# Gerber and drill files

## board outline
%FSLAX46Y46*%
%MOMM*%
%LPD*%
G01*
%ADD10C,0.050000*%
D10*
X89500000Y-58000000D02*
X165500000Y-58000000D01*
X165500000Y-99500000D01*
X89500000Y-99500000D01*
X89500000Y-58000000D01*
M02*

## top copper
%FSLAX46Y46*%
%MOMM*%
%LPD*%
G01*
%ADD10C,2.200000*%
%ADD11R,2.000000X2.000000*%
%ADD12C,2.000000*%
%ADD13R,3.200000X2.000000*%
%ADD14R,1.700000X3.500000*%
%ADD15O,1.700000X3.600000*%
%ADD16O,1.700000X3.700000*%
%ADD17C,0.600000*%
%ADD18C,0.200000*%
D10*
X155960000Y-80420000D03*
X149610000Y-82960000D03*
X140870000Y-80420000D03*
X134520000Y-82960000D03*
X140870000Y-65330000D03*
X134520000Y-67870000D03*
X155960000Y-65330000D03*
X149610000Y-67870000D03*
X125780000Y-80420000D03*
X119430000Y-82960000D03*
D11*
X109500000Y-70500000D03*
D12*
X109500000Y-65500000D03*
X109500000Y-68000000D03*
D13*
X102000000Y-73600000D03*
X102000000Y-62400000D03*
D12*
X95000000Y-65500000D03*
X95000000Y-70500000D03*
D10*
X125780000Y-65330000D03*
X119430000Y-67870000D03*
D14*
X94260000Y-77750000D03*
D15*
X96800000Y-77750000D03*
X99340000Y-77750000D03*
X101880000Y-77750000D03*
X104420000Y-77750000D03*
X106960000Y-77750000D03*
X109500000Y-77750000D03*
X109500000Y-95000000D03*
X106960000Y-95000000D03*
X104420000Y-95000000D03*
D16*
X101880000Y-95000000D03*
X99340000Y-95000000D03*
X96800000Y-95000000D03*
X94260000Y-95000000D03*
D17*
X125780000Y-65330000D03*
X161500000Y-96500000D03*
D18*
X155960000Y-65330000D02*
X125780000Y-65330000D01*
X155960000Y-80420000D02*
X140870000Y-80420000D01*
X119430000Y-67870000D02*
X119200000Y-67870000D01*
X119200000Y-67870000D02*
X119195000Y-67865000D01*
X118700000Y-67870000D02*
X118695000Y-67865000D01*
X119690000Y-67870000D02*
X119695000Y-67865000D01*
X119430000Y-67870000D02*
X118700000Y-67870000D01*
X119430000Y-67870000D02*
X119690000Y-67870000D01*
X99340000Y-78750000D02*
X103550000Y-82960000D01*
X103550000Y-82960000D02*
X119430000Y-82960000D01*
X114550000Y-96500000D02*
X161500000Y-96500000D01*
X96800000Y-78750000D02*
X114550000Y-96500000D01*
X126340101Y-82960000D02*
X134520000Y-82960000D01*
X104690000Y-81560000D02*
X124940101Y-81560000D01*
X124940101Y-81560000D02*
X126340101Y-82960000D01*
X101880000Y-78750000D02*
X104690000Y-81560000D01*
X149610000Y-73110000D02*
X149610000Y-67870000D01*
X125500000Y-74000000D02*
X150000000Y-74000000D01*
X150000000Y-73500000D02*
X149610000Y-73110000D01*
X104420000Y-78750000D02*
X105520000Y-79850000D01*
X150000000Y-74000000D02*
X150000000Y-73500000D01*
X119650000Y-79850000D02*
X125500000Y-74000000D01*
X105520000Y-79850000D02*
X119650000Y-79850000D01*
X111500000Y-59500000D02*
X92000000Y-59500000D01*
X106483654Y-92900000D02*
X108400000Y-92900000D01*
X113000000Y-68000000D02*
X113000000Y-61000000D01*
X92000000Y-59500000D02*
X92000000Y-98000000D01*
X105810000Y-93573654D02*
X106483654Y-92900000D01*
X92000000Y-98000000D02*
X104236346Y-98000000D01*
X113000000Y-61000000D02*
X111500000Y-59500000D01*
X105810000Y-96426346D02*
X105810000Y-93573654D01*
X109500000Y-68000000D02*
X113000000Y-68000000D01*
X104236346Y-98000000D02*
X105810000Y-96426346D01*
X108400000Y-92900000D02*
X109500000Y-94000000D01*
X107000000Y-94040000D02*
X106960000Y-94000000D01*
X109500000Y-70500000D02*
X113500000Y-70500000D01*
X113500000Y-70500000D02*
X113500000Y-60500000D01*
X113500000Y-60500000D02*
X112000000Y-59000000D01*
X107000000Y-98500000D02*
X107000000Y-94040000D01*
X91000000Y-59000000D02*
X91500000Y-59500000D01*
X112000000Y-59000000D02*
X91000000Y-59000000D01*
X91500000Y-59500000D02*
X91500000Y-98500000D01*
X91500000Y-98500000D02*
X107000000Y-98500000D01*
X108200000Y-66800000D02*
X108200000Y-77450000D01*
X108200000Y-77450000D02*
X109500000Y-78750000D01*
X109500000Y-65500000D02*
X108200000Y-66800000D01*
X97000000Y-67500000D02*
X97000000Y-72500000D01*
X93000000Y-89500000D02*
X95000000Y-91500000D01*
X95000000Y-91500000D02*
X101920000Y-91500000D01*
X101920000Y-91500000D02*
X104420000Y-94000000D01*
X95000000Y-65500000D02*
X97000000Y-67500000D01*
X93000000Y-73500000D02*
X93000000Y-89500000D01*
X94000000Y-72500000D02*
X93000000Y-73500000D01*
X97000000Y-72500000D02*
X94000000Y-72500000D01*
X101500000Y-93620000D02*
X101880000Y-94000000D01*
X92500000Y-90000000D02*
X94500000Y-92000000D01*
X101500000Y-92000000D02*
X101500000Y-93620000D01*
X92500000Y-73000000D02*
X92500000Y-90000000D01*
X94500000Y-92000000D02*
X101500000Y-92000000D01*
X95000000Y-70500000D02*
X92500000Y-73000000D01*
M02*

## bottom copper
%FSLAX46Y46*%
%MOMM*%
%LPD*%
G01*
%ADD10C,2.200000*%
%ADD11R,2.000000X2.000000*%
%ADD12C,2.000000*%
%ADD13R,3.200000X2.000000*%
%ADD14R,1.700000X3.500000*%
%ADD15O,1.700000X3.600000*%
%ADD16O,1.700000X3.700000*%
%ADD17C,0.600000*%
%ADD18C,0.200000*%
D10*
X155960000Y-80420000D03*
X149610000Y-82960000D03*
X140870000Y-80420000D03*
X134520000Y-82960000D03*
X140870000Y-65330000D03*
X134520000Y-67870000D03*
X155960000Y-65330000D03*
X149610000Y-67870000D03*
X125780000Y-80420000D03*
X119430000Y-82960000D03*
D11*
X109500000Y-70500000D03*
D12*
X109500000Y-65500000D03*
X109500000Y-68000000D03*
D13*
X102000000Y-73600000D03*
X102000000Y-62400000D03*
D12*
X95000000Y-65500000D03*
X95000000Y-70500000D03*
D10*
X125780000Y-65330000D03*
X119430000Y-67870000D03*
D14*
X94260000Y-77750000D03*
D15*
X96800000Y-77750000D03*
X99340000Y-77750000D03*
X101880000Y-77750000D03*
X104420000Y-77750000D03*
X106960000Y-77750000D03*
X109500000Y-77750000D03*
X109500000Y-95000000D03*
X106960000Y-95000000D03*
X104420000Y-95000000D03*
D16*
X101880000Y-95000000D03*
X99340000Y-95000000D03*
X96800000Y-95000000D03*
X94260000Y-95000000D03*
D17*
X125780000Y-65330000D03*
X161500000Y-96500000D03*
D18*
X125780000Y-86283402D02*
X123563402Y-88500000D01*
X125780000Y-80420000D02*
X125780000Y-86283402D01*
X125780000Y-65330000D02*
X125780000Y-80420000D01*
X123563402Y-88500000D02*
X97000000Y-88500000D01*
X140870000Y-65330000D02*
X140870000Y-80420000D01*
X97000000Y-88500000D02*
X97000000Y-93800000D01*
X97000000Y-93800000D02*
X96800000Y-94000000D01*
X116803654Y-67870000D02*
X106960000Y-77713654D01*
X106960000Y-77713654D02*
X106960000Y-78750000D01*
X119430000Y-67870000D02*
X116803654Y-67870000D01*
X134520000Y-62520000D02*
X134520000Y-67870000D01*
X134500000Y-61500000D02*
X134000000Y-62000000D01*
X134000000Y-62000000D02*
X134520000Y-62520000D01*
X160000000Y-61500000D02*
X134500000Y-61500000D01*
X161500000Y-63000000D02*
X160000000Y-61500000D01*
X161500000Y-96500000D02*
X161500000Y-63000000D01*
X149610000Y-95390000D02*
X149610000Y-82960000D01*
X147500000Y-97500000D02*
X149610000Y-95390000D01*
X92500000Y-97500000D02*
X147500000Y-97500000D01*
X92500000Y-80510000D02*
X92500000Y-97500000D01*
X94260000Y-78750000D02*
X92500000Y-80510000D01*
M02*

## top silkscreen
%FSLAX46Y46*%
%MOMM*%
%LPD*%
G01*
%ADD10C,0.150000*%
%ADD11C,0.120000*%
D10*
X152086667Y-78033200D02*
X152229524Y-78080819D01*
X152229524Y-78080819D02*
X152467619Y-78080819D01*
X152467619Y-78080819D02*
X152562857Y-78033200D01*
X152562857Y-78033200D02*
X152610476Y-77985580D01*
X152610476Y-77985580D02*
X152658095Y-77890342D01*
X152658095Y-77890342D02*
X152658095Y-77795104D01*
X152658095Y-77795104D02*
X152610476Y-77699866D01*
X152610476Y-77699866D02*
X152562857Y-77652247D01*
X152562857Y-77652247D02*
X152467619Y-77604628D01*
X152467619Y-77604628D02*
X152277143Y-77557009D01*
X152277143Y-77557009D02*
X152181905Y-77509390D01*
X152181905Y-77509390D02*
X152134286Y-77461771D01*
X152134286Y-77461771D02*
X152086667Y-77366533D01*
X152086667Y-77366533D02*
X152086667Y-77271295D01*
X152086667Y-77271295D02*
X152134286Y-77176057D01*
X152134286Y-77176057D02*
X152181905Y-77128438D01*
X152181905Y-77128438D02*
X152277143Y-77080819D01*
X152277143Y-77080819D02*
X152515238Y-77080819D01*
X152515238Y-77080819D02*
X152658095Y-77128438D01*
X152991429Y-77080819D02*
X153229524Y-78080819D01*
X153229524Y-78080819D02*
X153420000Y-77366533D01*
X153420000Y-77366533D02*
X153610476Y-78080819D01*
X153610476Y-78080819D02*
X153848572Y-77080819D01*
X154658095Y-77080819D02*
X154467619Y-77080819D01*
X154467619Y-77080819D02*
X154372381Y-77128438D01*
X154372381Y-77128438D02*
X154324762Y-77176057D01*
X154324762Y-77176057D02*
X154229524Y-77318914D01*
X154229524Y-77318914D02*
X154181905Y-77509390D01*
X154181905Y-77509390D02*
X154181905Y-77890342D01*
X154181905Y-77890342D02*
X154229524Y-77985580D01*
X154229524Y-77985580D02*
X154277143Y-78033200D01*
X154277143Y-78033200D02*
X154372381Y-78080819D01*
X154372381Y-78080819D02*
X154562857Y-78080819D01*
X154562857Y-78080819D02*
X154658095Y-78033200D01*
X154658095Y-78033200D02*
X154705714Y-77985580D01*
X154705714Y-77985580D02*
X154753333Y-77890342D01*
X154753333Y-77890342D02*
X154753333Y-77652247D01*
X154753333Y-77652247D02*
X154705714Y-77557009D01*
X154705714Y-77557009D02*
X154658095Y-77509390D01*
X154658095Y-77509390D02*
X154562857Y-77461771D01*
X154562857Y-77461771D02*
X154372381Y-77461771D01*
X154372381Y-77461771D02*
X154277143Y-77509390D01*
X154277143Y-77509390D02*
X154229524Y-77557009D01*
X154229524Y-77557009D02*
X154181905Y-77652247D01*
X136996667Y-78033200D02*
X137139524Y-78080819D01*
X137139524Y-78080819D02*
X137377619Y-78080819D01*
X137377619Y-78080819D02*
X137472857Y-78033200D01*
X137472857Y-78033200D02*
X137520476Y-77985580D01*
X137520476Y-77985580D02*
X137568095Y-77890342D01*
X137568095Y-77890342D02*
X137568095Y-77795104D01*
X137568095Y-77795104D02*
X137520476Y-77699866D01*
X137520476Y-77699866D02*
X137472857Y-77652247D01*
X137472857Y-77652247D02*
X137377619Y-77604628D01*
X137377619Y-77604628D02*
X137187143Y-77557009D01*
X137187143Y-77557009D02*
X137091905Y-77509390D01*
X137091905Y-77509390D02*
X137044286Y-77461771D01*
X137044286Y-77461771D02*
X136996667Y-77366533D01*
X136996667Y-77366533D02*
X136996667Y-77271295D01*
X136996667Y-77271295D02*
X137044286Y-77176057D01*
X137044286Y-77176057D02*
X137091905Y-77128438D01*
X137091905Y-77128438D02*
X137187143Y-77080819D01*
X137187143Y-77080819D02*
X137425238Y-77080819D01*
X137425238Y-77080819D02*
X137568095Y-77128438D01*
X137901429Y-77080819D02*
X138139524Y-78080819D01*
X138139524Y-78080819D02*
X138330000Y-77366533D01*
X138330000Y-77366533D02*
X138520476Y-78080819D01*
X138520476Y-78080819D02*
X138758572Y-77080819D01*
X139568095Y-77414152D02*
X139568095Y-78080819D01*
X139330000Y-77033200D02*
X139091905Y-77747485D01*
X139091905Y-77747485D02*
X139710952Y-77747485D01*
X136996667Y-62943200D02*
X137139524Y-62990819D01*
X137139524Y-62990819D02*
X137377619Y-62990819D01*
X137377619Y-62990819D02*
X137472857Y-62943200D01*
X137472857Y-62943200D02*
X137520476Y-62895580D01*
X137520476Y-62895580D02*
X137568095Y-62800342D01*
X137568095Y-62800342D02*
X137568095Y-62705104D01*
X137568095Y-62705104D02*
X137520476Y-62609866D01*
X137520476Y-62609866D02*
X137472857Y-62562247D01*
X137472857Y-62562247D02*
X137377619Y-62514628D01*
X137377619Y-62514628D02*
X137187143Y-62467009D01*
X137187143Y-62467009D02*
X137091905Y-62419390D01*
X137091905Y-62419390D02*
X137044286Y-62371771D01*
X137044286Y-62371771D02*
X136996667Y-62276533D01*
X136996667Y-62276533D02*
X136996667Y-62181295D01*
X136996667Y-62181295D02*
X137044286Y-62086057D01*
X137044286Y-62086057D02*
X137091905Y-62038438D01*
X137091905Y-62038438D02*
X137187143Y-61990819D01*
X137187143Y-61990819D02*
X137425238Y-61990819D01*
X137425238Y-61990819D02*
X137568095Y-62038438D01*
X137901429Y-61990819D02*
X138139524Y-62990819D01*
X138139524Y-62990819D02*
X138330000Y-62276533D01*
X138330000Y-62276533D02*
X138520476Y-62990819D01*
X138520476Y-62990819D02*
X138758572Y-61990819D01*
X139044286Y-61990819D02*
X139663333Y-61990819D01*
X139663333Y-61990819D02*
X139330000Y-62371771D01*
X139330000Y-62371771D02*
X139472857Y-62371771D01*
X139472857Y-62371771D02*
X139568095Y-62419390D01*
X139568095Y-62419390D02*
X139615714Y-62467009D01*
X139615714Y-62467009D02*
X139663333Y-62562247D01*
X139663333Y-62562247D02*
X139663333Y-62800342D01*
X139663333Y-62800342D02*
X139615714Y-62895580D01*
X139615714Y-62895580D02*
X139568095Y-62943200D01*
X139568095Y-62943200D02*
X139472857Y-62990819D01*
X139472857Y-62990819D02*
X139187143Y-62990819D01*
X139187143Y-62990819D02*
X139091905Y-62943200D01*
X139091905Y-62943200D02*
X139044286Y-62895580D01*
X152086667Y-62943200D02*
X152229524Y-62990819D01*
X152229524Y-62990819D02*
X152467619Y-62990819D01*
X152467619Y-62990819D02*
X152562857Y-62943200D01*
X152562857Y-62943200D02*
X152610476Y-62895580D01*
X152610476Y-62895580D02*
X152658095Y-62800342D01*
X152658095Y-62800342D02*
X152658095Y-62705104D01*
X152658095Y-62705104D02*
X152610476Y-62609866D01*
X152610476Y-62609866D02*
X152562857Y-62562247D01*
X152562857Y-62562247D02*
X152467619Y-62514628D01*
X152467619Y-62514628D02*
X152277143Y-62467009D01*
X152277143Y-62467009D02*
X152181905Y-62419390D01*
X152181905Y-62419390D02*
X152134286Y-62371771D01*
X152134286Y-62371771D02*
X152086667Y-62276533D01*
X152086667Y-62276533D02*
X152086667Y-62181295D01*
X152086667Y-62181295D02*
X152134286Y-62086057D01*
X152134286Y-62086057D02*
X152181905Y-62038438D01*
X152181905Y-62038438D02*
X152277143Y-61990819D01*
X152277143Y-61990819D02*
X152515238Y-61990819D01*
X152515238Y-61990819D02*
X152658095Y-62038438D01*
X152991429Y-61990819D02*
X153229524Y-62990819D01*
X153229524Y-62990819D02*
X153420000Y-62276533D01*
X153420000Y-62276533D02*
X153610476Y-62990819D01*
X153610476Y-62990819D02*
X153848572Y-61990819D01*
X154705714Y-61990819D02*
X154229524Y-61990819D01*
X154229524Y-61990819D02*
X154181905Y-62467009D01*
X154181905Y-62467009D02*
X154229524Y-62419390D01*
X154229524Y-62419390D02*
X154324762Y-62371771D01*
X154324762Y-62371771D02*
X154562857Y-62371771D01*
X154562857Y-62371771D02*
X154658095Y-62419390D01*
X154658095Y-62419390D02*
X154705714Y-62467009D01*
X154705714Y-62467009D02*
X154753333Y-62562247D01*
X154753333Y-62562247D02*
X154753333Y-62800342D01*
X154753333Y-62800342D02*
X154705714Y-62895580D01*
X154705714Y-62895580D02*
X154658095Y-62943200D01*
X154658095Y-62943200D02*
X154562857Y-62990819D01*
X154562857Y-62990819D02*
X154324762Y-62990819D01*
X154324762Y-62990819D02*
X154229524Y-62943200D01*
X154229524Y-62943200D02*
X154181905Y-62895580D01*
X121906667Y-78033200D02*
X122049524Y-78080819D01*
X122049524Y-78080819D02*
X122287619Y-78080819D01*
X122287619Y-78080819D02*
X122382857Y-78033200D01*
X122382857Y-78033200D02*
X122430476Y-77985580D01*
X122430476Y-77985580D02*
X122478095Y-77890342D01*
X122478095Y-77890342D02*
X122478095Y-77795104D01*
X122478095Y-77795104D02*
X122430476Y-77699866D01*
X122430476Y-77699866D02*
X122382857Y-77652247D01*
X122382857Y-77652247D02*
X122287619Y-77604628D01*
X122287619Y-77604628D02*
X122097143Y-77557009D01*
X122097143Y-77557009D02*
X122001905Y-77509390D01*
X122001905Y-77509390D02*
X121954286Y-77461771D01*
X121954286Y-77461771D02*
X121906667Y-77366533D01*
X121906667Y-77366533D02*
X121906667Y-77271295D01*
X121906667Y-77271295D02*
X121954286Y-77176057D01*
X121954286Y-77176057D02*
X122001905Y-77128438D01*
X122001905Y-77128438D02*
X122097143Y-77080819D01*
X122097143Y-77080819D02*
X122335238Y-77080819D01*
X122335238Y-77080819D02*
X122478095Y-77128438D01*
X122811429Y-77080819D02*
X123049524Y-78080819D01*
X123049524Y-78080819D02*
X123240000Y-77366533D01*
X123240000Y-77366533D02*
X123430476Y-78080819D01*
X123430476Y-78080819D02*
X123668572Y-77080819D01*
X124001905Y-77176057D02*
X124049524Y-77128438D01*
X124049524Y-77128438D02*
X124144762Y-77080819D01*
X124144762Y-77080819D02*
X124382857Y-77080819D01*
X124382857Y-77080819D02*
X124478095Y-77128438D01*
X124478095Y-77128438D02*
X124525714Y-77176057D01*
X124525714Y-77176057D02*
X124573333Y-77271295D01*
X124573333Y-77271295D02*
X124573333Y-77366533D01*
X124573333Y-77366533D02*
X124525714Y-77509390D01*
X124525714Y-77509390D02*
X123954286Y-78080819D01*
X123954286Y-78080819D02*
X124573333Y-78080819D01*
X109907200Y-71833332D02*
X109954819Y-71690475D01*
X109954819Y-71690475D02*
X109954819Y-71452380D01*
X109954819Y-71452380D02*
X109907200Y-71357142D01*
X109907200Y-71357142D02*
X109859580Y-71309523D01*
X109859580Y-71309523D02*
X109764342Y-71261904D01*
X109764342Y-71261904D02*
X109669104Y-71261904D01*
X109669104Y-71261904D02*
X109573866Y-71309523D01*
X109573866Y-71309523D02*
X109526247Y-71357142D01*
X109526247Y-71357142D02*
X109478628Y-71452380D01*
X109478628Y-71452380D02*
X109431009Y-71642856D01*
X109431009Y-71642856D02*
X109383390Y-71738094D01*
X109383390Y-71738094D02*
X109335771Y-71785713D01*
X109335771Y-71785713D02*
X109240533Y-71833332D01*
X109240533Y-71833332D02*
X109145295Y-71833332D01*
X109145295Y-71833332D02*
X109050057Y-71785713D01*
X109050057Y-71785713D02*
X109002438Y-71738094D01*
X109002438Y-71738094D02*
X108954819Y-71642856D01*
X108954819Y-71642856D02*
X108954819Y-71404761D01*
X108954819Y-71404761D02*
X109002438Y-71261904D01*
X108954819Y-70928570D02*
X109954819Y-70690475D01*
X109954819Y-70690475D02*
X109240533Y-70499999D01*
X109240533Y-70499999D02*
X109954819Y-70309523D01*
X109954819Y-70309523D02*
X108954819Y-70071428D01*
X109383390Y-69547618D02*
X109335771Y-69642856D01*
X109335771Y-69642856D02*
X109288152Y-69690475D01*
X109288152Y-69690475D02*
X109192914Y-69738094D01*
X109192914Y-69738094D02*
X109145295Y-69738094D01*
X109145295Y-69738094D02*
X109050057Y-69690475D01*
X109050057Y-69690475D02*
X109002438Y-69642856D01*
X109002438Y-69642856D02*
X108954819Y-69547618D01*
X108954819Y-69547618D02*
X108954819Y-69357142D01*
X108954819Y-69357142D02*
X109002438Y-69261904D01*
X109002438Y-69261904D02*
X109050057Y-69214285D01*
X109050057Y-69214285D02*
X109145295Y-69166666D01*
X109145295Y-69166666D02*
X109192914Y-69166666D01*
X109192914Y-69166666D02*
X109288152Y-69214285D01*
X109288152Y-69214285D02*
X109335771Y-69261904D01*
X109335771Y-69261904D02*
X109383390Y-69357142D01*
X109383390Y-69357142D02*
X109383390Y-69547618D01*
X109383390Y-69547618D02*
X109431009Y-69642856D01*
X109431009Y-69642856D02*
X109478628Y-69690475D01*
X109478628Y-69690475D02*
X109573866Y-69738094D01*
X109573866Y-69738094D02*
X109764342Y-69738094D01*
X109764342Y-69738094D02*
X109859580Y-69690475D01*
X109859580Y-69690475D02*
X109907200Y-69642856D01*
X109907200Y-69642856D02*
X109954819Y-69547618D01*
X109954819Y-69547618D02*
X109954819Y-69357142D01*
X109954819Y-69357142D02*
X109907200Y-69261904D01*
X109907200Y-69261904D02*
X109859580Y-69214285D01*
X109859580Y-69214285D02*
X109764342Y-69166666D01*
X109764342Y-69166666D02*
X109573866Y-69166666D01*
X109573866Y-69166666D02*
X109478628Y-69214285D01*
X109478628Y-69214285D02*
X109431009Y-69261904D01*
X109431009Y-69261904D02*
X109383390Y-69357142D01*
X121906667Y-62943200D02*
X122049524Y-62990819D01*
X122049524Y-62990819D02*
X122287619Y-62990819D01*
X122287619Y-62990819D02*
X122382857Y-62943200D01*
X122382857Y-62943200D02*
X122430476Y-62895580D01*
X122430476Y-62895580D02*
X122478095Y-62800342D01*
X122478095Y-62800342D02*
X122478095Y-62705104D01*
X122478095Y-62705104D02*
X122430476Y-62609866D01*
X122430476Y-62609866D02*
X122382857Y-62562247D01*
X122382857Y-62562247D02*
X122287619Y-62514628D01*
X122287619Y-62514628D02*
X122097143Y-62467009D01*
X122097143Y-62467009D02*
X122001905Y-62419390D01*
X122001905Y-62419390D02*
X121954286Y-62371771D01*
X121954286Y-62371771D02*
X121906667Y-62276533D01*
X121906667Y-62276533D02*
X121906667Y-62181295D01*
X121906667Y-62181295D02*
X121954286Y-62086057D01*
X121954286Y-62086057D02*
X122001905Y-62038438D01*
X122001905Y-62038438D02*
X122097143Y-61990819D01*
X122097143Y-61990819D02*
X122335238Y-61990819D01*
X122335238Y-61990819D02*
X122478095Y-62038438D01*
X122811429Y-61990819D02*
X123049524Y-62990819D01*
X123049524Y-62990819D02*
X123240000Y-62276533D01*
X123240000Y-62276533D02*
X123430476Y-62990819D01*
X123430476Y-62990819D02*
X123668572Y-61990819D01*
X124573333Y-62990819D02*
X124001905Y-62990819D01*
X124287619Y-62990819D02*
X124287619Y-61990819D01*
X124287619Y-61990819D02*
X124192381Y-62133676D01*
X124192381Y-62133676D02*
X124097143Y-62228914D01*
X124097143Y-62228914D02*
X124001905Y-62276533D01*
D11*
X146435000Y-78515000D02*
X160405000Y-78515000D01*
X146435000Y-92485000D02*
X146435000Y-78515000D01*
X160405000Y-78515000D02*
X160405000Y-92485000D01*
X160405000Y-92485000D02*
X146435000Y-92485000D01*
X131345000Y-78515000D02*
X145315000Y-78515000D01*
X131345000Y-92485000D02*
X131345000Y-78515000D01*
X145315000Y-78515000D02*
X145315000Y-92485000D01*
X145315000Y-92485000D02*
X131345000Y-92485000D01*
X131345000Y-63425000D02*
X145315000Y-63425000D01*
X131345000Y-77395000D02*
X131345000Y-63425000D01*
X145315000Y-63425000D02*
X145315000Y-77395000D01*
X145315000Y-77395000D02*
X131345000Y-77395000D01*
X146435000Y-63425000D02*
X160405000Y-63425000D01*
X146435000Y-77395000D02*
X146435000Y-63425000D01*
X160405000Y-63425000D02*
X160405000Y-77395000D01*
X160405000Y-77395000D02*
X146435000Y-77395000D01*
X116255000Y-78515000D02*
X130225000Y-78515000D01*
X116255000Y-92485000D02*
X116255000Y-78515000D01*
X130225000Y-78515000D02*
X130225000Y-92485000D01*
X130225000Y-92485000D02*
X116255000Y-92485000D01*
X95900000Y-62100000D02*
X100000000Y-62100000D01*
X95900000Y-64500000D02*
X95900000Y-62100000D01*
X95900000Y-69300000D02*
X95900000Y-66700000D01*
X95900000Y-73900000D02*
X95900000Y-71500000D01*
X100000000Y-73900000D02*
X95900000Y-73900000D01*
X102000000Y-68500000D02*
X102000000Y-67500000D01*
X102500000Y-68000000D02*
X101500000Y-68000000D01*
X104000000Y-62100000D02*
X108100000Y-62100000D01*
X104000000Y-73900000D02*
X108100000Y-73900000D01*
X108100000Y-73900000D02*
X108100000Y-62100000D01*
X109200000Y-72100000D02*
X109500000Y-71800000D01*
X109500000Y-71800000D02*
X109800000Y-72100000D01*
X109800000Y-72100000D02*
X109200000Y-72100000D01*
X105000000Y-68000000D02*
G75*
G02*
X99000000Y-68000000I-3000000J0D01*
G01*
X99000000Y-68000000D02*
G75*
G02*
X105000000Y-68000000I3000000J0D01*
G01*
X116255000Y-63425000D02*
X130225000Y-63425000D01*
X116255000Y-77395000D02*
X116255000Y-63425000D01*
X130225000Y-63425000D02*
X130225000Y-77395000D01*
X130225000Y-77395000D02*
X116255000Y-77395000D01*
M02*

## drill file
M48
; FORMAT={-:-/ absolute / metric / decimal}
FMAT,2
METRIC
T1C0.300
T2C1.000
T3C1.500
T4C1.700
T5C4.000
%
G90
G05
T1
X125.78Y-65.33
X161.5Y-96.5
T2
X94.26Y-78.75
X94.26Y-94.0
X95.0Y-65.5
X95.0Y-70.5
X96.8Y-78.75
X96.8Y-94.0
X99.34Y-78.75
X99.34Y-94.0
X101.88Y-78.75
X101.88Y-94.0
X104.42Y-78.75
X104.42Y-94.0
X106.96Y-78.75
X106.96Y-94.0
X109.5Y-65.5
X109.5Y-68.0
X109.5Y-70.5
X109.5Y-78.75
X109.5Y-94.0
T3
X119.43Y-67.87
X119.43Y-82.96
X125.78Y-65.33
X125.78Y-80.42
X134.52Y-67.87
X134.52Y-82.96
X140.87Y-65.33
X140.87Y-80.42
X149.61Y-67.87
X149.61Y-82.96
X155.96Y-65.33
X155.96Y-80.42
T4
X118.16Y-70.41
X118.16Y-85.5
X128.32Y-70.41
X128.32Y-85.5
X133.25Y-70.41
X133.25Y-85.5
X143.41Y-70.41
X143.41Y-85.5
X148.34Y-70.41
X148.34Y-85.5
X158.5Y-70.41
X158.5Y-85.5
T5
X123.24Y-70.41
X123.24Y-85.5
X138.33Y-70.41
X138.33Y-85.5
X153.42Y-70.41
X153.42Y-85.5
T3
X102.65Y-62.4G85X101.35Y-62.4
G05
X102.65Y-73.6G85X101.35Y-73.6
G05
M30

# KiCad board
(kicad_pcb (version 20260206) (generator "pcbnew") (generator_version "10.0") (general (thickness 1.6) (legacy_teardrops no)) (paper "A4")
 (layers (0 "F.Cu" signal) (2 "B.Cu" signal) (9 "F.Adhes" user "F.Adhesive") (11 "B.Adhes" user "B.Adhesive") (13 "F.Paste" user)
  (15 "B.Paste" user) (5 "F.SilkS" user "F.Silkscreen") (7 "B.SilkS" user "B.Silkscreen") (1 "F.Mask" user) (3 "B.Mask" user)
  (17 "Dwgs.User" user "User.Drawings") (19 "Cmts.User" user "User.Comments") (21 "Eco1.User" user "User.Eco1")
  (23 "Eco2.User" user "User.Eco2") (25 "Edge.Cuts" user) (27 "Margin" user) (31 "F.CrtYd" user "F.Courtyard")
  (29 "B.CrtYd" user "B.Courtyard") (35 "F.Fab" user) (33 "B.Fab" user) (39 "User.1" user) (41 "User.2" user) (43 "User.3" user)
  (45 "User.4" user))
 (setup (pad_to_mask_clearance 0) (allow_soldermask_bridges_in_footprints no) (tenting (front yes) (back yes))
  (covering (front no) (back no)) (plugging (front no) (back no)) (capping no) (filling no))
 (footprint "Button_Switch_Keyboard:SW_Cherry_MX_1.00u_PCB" (layer "F.Cu") (at 155.96 80.42)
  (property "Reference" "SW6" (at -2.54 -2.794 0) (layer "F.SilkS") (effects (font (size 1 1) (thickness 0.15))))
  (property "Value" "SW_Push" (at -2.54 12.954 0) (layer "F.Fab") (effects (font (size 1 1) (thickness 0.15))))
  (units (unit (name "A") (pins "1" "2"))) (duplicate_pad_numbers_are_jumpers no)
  (fp_line (start -9.525 -1.905) (end 4.445 -1.905) (stroke (width 0.12) (type solid)) (layer "F.SilkS"))
  (fp_line (start -9.525 12.065) (end -9.525 -1.905) (stroke (width 0.12) (type solid)) (layer "F.SilkS"))
  (fp_line (start 4.445 -1.905) (end 4.445 12.065) (stroke (width 0.12) (type solid)) (layer "F.SilkS"))
  (fp_line (start 4.445 12.065) (end -9.525 12.065) (stroke (width 0.12) (type solid)) (layer "F.SilkS"))
  (pad "" np_thru_hole circle (at -7.62 5.08) (size 1.7 1.7) (drill 1.7) (layers "*.Cu" "*.Mask"))
  (pad "" np_thru_hole circle (at -2.54 5.08) (size 4 4) (drill 4) (layers "*.Cu" "*.Mask"))
  (pad "" np_thru_hole circle (at 2.54 5.08) (size 1.7 1.7) (drill 1.7) (layers "*.Cu" "*.Mask"))
  (pad "1" thru_hole circle (at 0 0) (size 2.2 2.2) (drill 1.5) (layers "*.Cu" "*.Mask") (remove_unused_layers no) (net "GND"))
  (pad "2" thru_hole circle (at -6.35 2.54) (size 2.2 2.2) (drill 1.5) (layers "*.Cu" "*.Mask") (remove_unused_layers no)
   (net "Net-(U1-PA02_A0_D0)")))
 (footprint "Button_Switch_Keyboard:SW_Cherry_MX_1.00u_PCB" (layer "F.Cu") (at 140.87 80.42)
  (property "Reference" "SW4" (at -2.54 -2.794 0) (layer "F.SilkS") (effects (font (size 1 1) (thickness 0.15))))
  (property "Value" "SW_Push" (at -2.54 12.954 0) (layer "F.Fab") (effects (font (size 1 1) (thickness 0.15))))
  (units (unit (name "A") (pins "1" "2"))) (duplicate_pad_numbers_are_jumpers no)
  (fp_line (start -9.525 -1.905) (end 4.445 -1.905) (stroke (width 0.12) (type solid)) (layer "F.SilkS"))
  (fp_line (start -9.525 12.065) (end -9.525 -1.905) (stroke (width 0.12) (type solid)) (layer "F.SilkS"))
  (fp_line (start 4.445 -1.905) (end 4.445 12.065) (stroke (width 0.12) (type solid)) (layer "F.SilkS"))
  (fp_line (start 4.445 12.065) (end -9.525 12.065) (stroke (width 0.12) (type solid)) (layer "F.SilkS"))
  (pad "" np_thru_hole circle (at -7.62 5.08) (size 1.7 1.7) (drill 1.7) (layers "*.Cu" "*.Mask"))
  (pad "" np_thru_hole circle (at -2.54 5.08) (size 4 4) (drill 4) (layers "*.Cu" "*.Mask"))
  (pad "" np_thru_hole circle (at 2.54 5.08) (size 1.7 1.7) (drill 1.7) (layers "*.Cu" "*.Mask"))
  (pad "1" thru_hole circle (at 0 0) (size 2.2 2.2) (drill 1.5) (layers "*.Cu" "*.Mask") (remove_unused_layers no) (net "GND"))
  (pad "2" thru_hole circle (at -6.35 2.54) (size 2.2 2.2) (drill 1.5) (layers "*.Cu" "*.Mask") (remove_unused_layers no)
   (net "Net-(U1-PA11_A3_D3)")))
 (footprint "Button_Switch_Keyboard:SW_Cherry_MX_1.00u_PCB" (layer "F.Cu") (at 140.87 65.33)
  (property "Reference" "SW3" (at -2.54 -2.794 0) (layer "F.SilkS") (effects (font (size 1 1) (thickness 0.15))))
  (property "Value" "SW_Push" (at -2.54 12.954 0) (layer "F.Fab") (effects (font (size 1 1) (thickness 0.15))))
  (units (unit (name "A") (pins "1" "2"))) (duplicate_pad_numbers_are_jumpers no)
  (fp_line (start -9.525 -1.905) (end 4.445 -1.905) (stroke (width 0.12) (type solid)) (layer "F.SilkS"))
  (fp_line (start -9.525 12.065) (end -9.525 -1.905) (stroke (width 0.12) (type solid)) (layer "F.SilkS"))
  (fp_line (start 4.445 -1.905) (end 4.445 12.065) (stroke (width 0.12) (type solid)) (layer "F.SilkS"))
  (fp_line (start 4.445 12.065) (end -9.525 12.065) (stroke (width 0.12) (type solid)) (layer "F.SilkS"))
  (pad "" np_thru_hole circle (at -7.62 5.08) (size 1.7 1.7) (drill 1.7) (layers "*.Cu" "*.Mask"))
  (pad "" np_thru_hole circle (at -2.54 5.08) (size 4 4) (drill 4) (layers "*.Cu" "*.Mask"))
  (pad "" np_thru_hole circle (at 2.54 5.08) (size 1.7 1.7) (drill 1.7) (layers "*.Cu" "*.Mask"))
  (pad "1" thru_hole circle (at 0 0) (size 2.2 2.2) (drill 1.5) (layers "*.Cu" "*.Mask") (remove_unused_layers no) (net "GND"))
  (pad "2" thru_hole circle (at -6.35 2.54) (size 2.2 2.2) (drill 1.5) (layers "*.Cu" "*.Mask") (remove_unused_layers no)
   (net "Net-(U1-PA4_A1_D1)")))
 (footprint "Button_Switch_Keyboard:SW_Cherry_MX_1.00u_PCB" (layer "F.Cu") (at 155.96 65.33)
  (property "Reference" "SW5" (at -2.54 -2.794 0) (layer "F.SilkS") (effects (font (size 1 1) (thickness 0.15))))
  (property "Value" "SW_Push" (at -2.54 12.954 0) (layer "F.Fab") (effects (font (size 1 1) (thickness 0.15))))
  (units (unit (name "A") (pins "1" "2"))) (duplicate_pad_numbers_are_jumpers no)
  (fp_line (start -9.525 -1.905) (end 4.445 -1.905) (stroke (width 0.12) (type solid)) (layer "F.SilkS"))
  (fp_line (start -9.525 12.065) (end -9.525 -1.905) (stroke (width 0.12) (type solid)) (layer "F.SilkS"))
  (fp_line (start 4.445 -1.905) (end 4.445 12.065) (stroke (width 0.12) (type solid)) (layer "F.SilkS"))
  (fp_line (start 4.445 12.065) (end -9.525 12.065) (stroke (width 0.12) (type solid)) (layer "F.SilkS"))
  (pad "" np_thru_hole circle (at -7.62 5.08) (size 1.7 1.7) (drill 1.7) (layers "*.Cu" "*.Mask"))
  (pad "" np_thru_hole circle (at -2.54 5.08) (size 4 4) (drill 4) (layers "*.Cu" "*.Mask"))
  (pad "" np_thru_hole circle (at 2.54 5.08) (size 1.7 1.7) (drill 1.7) (layers "*.Cu" "*.Mask"))
  (pad "1" thru_hole circle (at 0 0) (size 2.2 2.2) (drill 1.5) (layers "*.Cu" "*.Mask") (remove_unused_layers no) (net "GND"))
  (pad "2" thru_hole circle (at -6.35 2.54) (size 2.2 2.2) (drill 1.5) (layers "*.Cu" "*.Mask") (remove_unused_layers no)
   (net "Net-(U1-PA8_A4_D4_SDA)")))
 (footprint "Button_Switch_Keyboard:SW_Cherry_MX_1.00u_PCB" (layer "F.Cu") (at 125.78 80.42)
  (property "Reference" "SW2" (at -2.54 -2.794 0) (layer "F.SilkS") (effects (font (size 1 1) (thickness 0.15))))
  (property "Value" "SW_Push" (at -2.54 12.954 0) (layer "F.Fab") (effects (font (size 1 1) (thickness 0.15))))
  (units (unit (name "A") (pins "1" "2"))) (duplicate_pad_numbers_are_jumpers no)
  (fp_line (start -9.525 -1.905) (end 4.445 -1.905) (stroke (width 0.12) (type solid)) (layer "F.SilkS"))
  (fp_line (start -9.525 12.065) (end -9.525 -1.905) (stroke (width 0.12) (type solid)) (layer "F.SilkS"))
  (fp_line (start 4.445 -1.905) (end 4.445 12.065) (stroke (width 0.12) (type solid)) (layer "F.SilkS"))
  (fp_line (start 4.445 12.065) (end -9.525 12.065) (stroke (width 0.12) (type solid)) (layer "F.SilkS"))
  (pad "" np_thru_hole circle (at -7.62 5.08) (size 1.7 1.7) (drill 1.7) (layers "*.Cu" "*.Mask"))
  (pad "" np_thru_hole circle (at -2.54 5.08) (size 4 4) (drill 4) (layers "*.Cu" "*.Mask"))
  (pad "" np_thru_hole circle (at 2.54 5.08) (size 1.7 1.7) (drill 1.7) (layers "*.Cu" "*.Mask"))
  (pad "1" thru_hole circle (at 0 0) (size 2.2 2.2) (drill 1.5) (layers "*.Cu" "*.Mask") (remove_unused_layers no) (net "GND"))
  (pad "2" thru_hole circle (at -6.35 2.54) (size 2.2 2.2) (drill 1.5) (layers "*.Cu" "*.Mask") (remove_unused_layers no)
   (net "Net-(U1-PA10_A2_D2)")))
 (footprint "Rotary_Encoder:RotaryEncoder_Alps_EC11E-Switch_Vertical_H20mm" (layer "F.Cu") (at 109.5 70.5 180)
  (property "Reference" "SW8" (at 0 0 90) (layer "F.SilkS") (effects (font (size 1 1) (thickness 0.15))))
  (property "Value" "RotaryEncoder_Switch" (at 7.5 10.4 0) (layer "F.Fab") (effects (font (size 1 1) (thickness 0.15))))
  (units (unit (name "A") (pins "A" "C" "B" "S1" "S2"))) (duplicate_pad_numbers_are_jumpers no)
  (fp_line (start 13.6 8.4) (end 9.5 8.4) (stroke (width 0.12) (type solid)) (layer "F.SilkS"))
  (fp_line (start 13.6 6) (end 13.6 8.4) (stroke (width 0.12) (type solid)) (layer "F.SilkS"))
  (fp_line (start 13.6 1.2) (end 13.6 3.8) (stroke (width 0.12) (type solid)) (layer "F.SilkS"))
  (fp_line (start 13.6 -3.4) (end 13.6 -1) (stroke (width 0.12) (type solid)) (layer "F.SilkS"))
  (fp_line (start 9.5 -3.4) (end 13.6 -3.4) (stroke (width 0.12) (type solid)) (layer "F.SilkS"))
  (fp_line (start 7.5 2) (end 7.5 3) (stroke (width 0.12) (type solid)) (layer "F.SilkS"))
  (fp_line (start 7 2.5) (end 8 2.5) (stroke (width 0.12) (type solid)) (layer "F.SilkS"))
  (fp_line (start 5.5 8.4) (end 1.4 8.4) (stroke (width 0.12) (type solid)) (layer "F.SilkS"))
  (fp_line (start 5.5 -3.4) (end 1.4 -3.4) (stroke (width 0.12) (type solid)) (layer "F.SilkS"))
  (fp_line (start 1.4 -3.4) (end 1.4 8.4) (stroke (width 0.12) (type solid)) (layer "F.SilkS"))
  (fp_line (start 0.3 -1.6) (end 0 -1.3) (stroke (width 0.12) (type solid)) (layer "F.SilkS"))
  (fp_line (start 0 -1.3) (end -0.3 -1.6) (stroke (width 0.12) (type solid)) (layer "F.SilkS"))
  (fp_line (start -0.3 -1.6) (end 0.3 -1.6) (stroke (width 0.12) (type solid)) (layer "F.SilkS"))
  (fp_circle (center 7.5 2.5) (end 10.5 2.5) (stroke (width 0.12) (type solid)) (fill no) (layer "F.SilkS"))
  (pad "A" thru_hole rect (at 0 0 180) (size 2 2) (drill 1) (layers "*.Cu" "*.Mask") (remove_unused_layers no)
   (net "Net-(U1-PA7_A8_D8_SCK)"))
  (pad "B" thru_hole circle (at 0 5 180) (size 2 2) (drill 1) (layers "*.Cu" "*.Mask") (remove_unused_layers no)
   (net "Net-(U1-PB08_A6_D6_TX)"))
  (pad "C" thru_hole circle (at 0 2.5 180) (size 2 2) (drill 1) (layers "*.Cu" "*.Mask") (remove_unused_layers no)
   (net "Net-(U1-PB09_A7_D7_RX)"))
  (pad "MP" thru_hole rect (at 7.5 -3.1 180) (size 3.2 2) (drill oval 2.8 1.5) (layers "*.Cu" "*.Mask") (remove_unused_layers no))
  (pad "MP" thru_hole rect (at 7.5 8.1 180) (size 3.2 2) (drill oval 2.8 1.5) (layers "*.Cu" "*.Mask") (remove_unused_layers no))
  (pad "S1" thru_hole circle (at 14.5 5 180) (size 2 2) (drill 1) (layers "*.Cu" "*.Mask") (remove_unused_layers no)
   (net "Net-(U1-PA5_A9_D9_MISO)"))
  (pad "S2" thru_hole circle (at 14.5 0 180) (size 2 2) (drill 1) (layers "*.Cu" "*.Mask") (remove_unused_layers no)
   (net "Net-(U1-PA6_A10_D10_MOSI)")))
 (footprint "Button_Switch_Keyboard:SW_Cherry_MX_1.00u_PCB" (layer "F.Cu") (at 125.78 65.33)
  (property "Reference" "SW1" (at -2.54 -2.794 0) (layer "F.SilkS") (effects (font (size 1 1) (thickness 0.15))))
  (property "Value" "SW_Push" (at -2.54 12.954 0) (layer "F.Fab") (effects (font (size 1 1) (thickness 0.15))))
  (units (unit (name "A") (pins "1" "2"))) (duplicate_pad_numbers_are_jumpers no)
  (fp_line (start -9.525 -1.905) (end 4.445 -1.905) (stroke (width 0.12) (type solid)) (layer "F.SilkS"))
  (fp_line (start -9.525 12.065) (end -9.525 -1.905) (stroke (width 0.12) (type solid)) (layer "F.SilkS"))
  (fp_line (start 4.445 -1.905) (end 4.445 12.065) (stroke (width 0.12) (type solid)) (layer "F.SilkS"))
  (fp_line (start 4.445 12.065) (end -9.525 12.065) (stroke (width 0.12) (type solid)) (layer "F.SilkS"))
  (pad "" np_thru_hole circle (at -7.62 5.08) (size 1.7 1.7) (drill 1.7) (layers "*.Cu" "*.Mask"))
  (pad "" np_thru_hole circle (at -2.54 5.08) (size 4 4) (drill 4) (layers "*.Cu" "*.Mask"))
  (pad "" np_thru_hole circle (at 2.54 5.08) (size 1.7 1.7) (drill 1.7) (layers "*.Cu" "*.Mask"))
  (pad "1" thru_hole circle (at 0 0) (size 2.2 2.2) (drill 1.5) (layers "*.Cu" "*.Mask") (remove_unused_layers no) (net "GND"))
  (pad "2" thru_hole circle (at -6.35 2.54) (size 2.2 2.2) (drill 1.5) (layers "*.Cu" "*.Mask") (remove_unused_layers no)
   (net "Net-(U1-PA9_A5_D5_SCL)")))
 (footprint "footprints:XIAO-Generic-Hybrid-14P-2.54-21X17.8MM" (layer "B.Cu") (at 101.88 86.375 -90)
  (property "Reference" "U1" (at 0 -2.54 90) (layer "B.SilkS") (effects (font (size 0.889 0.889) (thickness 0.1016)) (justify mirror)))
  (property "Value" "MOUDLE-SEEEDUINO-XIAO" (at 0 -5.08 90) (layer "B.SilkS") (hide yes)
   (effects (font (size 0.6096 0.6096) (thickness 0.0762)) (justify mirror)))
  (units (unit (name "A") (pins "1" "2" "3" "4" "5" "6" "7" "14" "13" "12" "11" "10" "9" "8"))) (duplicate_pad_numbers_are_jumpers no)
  (pad "1" thru_hole rect (at -7.625 7.62 270) (size 3.5 1.7) (drill 1 (offset -1 0)) (layers "*.Cu" "*.Mask") (remove_unused_layers no)
   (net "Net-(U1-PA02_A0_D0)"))
  (pad "2" thru_hole oval (at -7.625 5.08 270) (size 3.6 1.7) (drill 1 (offset -1 0)) (layers "*.Cu" "*.Mask") (remove_unused_layers no)
   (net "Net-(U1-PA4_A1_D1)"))
  (pad "3" thru_hole oval (at -7.625 2.54 270) (size 3.6 1.7) (drill 1 (offset -1 0)) (layers "*.Cu" "*.Mask") (remove_unused_layers no)
   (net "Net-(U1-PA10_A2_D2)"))
  (pad "4" thru_hole oval (at -7.625 0 270) (size 3.6 1.7) (drill 1 (offset -1 0)) (layers "*.Cu" "*.Mask") (remove_unused_layers no)
   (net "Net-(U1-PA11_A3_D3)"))
  (pad "5" thru_hole oval (at -7.625 -2.54 270) (size 3.6 1.7) (drill 1 (offset -1 0)) (layers "*.Cu" "*.Mask") (remove_unused_layers no)
   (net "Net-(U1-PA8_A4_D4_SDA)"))
  (pad "6" thru_hole oval (at -7.625 -5.08 90) (size 3.6 1.7) (drill 1 (offset 1 0)) (layers "*.Cu" "*.Mask") (remove_unused_layers no)
   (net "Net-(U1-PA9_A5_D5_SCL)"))
  (pad "7" thru_hole oval (at -7.625 -7.62 270) (size 3.6 1.7) (drill 1 (offset -1 0)) (layers "*.Cu" "*.Mask") (remove_unused_layers no)
   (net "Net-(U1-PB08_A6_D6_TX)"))
  (pad "8" thru_hole oval (at 7.625 -7.62 270) (size 3.6 1.7) (drill 1 (offset 1 0)) (layers "*.Cu" "*.Mask") (remove_unused_layers no)
   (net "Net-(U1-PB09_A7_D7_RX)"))
  (pad "9" thru_hole oval (at 7.625 -5.08 270) (size 3.6 1.7) (drill 1 (offset 1 0)) (layers "*.Cu" "*.Mask") (remove_unused_layers no)
   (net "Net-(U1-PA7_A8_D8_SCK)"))
  (pad "10" thru_hole oval (at 7.625 -2.54 270) (size 3.6 1.7) (drill 1 (offset 1 0)) (layers "*.Cu" "*.Mask") (remove_unused_layers no)
   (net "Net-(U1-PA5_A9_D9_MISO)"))
  (pad "11" thru_hole oval (at 7.625 0 270) (size 3.7 1.7) (drill 1 (offset 1 0)) (layers "*.Cu" "*.Mask") (remove_unused_layers no)
   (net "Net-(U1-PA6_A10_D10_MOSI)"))
  (pad "12" thru_hole oval (at 7.625 2.54 270) (size 3.7 1.7) (drill 1 (offset 1 0)) (layers "*.Cu" "*.Mask") (remove_unused_layers no)
   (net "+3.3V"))
  (pad "13" thru_hole oval (at 7.625 5.08 270) (size 3.7 1.7) (drill 1 (offset 1 0)) (layers "*.Cu" "*.Mask") (remove_unused_layers no)
   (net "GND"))
  (pad "14" thru_hole oval (at 7.625 7.62 270) (size 3.7 1.7) (drill 1 (offset 1 0)) (layers "*.Cu" "*.Mask") (remove_unused_layers no)
   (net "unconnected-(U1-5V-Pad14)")))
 (gr_rect (start 89.5 58) (end 165.5 99.5) (stroke (width 0.05) (type default)) (fill no) (layer "Edge.Cuts"))
 (segment (start 155.96 65.33) (end 125.78 65.33) (width 0.2) (layer "F.Cu") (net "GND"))
 (segment (start 155.96 80.42) (end 140.87 80.42) (width 0.2) (layer "F.Cu") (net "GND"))
 (via (at 125.78 65.33) (size 0.6) (drill 0.3) (layers "F.Cu" "B.Cu") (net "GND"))
 (segment (start 125.78 86.283402) (end 123.563402 88.5) (width 0.2) (layer "B.Cu") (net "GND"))
 (segment (start 125.78 80.42) (end 125.78 86.283402) (width 0.2) (layer "B.Cu") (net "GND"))
 (segment (start 125.78 65.33) (end 125.78 80.42) (width 0.2) (layer "B.Cu") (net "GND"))
 (segment (start 123.563402 88.5) (end 97 88.5) (width 0.2) (layer "B.Cu") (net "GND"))
 (segment (start 140.87 65.33) (end 140.87 80.42) (width 0.2) (layer "B.Cu") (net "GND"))
 (segment (start 97 88.5) (end 97 93.8) (width 0.2) (layer "B.Cu") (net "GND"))
 (segment (start 97 93.8) (end 96.8 94) (width 0.2) (layer "B.Cu") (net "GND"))
 (segment (start 119.43 67.87) (end 119.2 67.87) (width 0.2) (layer "F.Cu") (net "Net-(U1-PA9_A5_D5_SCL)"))
 (segment (start 119.2 67.87) (end 119.195 67.865) (width 0.2) (layer "F.Cu") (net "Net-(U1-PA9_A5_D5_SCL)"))
 (segment (start 118.7 67.87) (end 118.695 67.865) (width 0.2) (layer "F.Cu") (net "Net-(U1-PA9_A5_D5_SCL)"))
 (segment (start 119.69 67.87) (end 119.695 67.865) (width 0.2) (layer "F.Cu") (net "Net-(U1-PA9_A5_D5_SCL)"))
 (segment (start 119.43 67.87) (end 118.7 67.87) (width 0.2) (layer "F.Cu") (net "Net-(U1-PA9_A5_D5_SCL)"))
 (segment (start 119.43 67.87) (end 119.69 67.87) (width 0.2) (layer "F.Cu") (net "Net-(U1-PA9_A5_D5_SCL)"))
 (segment (start 116.803654 67.87) (end 106.96 77.713654) (width 0.2) (layer "B.Cu") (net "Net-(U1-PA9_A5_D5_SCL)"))
 (segment (start 106.96 77.713654) (end 106.96 78.75) (width 0.2) (layer "B.Cu") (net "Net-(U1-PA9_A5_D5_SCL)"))
 (segment (start 119.43 67.87) (end 116.803654 67.87) (width 0.2) (layer "B.Cu") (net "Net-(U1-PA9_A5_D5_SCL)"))
 (segment (start 99.34 78.75) (end 103.55 82.96) (width 0.2) (layer "F.Cu") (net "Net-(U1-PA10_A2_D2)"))
 (segment (start 103.55 82.96) (end 119.43 82.96) (width 0.2) (layer "F.Cu") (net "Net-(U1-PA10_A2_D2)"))
 (segment (start 114.55 96.5) (end 161.5 96.5) (width 0.2) (layer "F.Cu") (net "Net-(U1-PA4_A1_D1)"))
 (segment (start 96.8 78.75) (end 114.55 96.5) (width 0.2) (layer "F.Cu") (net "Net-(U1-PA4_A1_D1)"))
 (via (at 161.5 96.5) (size 0.6) (drill 0.3) (layers "F.Cu" "B.Cu") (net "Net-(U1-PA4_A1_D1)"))
 (segment (start 134.52 62.52) (end 134.52 67.87) (width 0.2) (layer "B.Cu") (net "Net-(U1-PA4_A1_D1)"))
 (segment (start 134.5 61.5) (end 134 62) (width 0.2) (layer "B.Cu") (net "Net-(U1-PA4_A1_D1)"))
 (segment (start 134 62) (end 134.52 62.52) (width 0.2) (layer "B.Cu") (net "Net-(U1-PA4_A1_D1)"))
 (segment (start 160 61.5) (end 134.5 61.5) (width 0.2) (layer "B.Cu") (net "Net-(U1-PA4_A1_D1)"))
 (segment (start 161.5 63) (end 160 61.5) (width 0.2) (layer "B.Cu") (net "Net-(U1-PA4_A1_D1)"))
 (segment (start 161.5 96.5) (end 161.5 63) (width 0.2) (layer "B.Cu") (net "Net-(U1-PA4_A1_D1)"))
 (segment (start 126.340101 82.96) (end 134.52 82.96) (width 0.2) (layer "F.Cu") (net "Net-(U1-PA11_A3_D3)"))
 (segment (start 104.69 81.56) (end 124.940101 81.56) (width 0.2) (layer "F.Cu") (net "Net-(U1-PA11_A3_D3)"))
 (segment (start 124.940101 81.56) (end 126.340101 82.96) (width 0.2) (layer "F.Cu") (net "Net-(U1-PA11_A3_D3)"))
 (segment (start 101.88 78.75) (end 104.69 81.56) (width 0.2) (layer "F.Cu") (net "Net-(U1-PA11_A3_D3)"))
 (segment (start 149.61 73.11) (end 149.61 67.87) (width 0.2) (layer "F.Cu") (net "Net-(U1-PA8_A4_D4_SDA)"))
 (segment (start 125.5 74) (end 150 74) (width 0.2) (layer "F.Cu") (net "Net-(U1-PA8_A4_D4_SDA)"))
 (segment (start 150 73.5) (end 149.61 73.11) (width 0.2) (layer "F.Cu") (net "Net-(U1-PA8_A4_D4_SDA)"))
 (segment (start 104.42 78.75) (end 105.52 79.85) (width 0.2) (layer "F.Cu") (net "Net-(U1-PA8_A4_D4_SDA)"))
 (segment (start 150 74) (end 150 73.5) (width 0.2) (layer "F.Cu") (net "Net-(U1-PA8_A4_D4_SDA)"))
 (segment (start 119.65 79.85) (end 125.5 74) (width 0.2) (layer "F.Cu") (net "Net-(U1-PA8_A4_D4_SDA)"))
 (segment (start 105.52 79.85) (end 119.65 79.85) (width 0.2) (layer "F.Cu") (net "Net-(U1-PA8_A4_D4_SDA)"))
 (segment (start 149.61 95.39) (end 149.61 82.96) (width 0.2) (layer "B.Cu") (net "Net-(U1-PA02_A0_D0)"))
 (segment (start 147.5 97.5) (end 149.61 95.39) (width 0.2) (layer "B.Cu") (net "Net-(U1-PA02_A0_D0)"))
 (segment (start 92.5 97.5) (end 147.5 97.5) (width 0.2) (layer "B.Cu") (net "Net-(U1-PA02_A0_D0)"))
 (segment (start 92.5 80.51) (end 92.5 97.5) (width 0.2) (layer "B.Cu") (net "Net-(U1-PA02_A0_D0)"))
 (segment (start 94.26 78.75) (end 92.5 80.51) (width 0.2) (layer "B.Cu") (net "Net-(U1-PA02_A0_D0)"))
 (segment (start 111.5 59.5) (end 92 59.5) (width 0.2) (layer "F.Cu") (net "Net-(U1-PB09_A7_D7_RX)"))
 (segment (start 106.483654 92.9) (end 108.4 92.9) (width 0.2) (layer "F.Cu") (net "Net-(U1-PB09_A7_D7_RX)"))
 (segment (start 113 68) (end 113 61) (width 0.2) (layer "F.Cu") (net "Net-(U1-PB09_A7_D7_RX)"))
 (segment (start 92 59.5) (end 92 98) (width 0.2) (layer "F.Cu") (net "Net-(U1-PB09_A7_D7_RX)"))
 (segment (start 105.81 93.573654) (end 106.483654 92.9) (width 0.2) (layer "F.Cu") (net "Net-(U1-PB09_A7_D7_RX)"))
 (segment (start 92 98) (end 104.236346 98) (width 0.2) (layer "F.Cu") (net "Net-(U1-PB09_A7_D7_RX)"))
 (segment (start 113 61) (end 111.5 59.5) (width 0.2) (layer "F.Cu") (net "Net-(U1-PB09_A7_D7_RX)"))
 (segment (start 105.81 96.426346) (end 105.81 93.573654) (width 0.2) (layer "F.Cu") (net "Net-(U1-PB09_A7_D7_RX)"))
 (segment (start 109.5 68) (end 113 68) (width 0.2) (layer "F.Cu") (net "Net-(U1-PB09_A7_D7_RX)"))
 (segment (start 104.236346 98) (end 105.81 96.426346) (width 0.2) (layer "F.Cu") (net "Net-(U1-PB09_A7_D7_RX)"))
 (segment (start 108.4 92.9) (end 109.5 94) (width 0.2) (layer "F.Cu") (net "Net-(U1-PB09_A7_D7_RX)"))
 (segment (start 107 94.04) (end 106.96 94) (width 0.2) (layer "F.Cu") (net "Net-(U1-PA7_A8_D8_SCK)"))
 (segment (start 109.5 70.5) (end 113.5 70.5) (width 0.2) (layer "F.Cu") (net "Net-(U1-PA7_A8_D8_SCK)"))
 (segment (start 113.5 70.5) (end 113.5 60.5) (width 0.2) (layer "F.Cu") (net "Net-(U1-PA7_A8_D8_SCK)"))
 (segment (start 113.5 60.5) (end 112 59) (width 0.2) (layer "F.Cu") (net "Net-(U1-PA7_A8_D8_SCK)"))
 (segment (start 107 98.5) (end 107 94.04) (width 0.2) (layer "F.Cu") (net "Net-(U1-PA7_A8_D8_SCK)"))
 (segment (start 91 59) (end 91.5 59.5) (width 0.2) (layer "F.Cu") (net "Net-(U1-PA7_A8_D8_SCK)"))
 (segment (start 112 59) (end 91 59) (width 0.2) (layer "F.Cu") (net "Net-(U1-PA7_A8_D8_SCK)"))
 (segment (start 91.5 59.5) (end 91.5 98.5) (width 0.2) (layer "F.Cu") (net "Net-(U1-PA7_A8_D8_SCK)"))
 (segment (start 91.5 98.5) (end 107 98.5) (width 0.2) (layer "F.Cu") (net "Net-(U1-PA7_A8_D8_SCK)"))
 (segment (start 108.2 66.8) (end 108.2 77.45) (width 0.2) (layer "F.Cu") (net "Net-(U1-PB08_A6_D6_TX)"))
 (segment (start 108.2 77.45) (end 109.5 78.75) (width 0.2) (layer "F.Cu") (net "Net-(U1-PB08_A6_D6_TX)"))
 (segment (start 109.5 65.5) (end 108.2 66.8) (width 0.2) (layer "F.Cu") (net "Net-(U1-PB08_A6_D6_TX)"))
 (segment (start 97 67.5) (end 97 72.5) (width 0.2) (layer "F.Cu") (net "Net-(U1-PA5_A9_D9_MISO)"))
 (segment (start 93 89.5) (end 95 91.5) (width 0.2) (layer "F.Cu") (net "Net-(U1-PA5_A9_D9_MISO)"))
 (segment (start 95 91.5) (end 101.92 91.5) (width 0.2) (layer "F.Cu") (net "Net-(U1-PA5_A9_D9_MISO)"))
 (segment (start 101.92 91.5) (end 104.42 94) (width 0.2) (layer "F.Cu") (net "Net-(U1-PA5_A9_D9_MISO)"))
 (segment (start 95 65.5) (end 97 67.5) (width 0.2) (layer "F.Cu") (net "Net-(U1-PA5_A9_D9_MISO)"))
 (segment (start 93 73.5) (end 93 89.5) (width 0.2) (layer "F.Cu") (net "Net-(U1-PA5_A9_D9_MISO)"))
 (segment (start 94 72.5) (end 93 73.5) (width 0.2) (layer "F.Cu") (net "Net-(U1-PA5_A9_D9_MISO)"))
 (segment (start 97 72.5) (end 94 72.5) (width 0.2) (layer "F.Cu") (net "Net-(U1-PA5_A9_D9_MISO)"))
 (segment (start 101.5 93.62) (end 101.88 94) (width 0.2) (layer "F.Cu") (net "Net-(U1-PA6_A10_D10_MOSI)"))
 (segment (start 92.5 90) (end 94.5 92) (width 0.2) (layer "F.Cu") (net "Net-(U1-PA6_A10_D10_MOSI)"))
 (segment (start 101.5 92) (end 101.5 93.62) (width 0.2) (layer "F.Cu") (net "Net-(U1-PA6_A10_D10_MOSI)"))
 (segment (start 92.5 73) (end 92.5 90) (width 0.2) (layer "F.Cu") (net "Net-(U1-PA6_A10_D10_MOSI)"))
 (segment (start 94.5 92) (end 101.5 92) (width 0.2) (layer "F.Cu") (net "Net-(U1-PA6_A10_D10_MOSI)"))
 (segment (start 95 70.5) (end 92.5 73) (width 0.2) (layer "F.Cu") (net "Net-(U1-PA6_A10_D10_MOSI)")))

